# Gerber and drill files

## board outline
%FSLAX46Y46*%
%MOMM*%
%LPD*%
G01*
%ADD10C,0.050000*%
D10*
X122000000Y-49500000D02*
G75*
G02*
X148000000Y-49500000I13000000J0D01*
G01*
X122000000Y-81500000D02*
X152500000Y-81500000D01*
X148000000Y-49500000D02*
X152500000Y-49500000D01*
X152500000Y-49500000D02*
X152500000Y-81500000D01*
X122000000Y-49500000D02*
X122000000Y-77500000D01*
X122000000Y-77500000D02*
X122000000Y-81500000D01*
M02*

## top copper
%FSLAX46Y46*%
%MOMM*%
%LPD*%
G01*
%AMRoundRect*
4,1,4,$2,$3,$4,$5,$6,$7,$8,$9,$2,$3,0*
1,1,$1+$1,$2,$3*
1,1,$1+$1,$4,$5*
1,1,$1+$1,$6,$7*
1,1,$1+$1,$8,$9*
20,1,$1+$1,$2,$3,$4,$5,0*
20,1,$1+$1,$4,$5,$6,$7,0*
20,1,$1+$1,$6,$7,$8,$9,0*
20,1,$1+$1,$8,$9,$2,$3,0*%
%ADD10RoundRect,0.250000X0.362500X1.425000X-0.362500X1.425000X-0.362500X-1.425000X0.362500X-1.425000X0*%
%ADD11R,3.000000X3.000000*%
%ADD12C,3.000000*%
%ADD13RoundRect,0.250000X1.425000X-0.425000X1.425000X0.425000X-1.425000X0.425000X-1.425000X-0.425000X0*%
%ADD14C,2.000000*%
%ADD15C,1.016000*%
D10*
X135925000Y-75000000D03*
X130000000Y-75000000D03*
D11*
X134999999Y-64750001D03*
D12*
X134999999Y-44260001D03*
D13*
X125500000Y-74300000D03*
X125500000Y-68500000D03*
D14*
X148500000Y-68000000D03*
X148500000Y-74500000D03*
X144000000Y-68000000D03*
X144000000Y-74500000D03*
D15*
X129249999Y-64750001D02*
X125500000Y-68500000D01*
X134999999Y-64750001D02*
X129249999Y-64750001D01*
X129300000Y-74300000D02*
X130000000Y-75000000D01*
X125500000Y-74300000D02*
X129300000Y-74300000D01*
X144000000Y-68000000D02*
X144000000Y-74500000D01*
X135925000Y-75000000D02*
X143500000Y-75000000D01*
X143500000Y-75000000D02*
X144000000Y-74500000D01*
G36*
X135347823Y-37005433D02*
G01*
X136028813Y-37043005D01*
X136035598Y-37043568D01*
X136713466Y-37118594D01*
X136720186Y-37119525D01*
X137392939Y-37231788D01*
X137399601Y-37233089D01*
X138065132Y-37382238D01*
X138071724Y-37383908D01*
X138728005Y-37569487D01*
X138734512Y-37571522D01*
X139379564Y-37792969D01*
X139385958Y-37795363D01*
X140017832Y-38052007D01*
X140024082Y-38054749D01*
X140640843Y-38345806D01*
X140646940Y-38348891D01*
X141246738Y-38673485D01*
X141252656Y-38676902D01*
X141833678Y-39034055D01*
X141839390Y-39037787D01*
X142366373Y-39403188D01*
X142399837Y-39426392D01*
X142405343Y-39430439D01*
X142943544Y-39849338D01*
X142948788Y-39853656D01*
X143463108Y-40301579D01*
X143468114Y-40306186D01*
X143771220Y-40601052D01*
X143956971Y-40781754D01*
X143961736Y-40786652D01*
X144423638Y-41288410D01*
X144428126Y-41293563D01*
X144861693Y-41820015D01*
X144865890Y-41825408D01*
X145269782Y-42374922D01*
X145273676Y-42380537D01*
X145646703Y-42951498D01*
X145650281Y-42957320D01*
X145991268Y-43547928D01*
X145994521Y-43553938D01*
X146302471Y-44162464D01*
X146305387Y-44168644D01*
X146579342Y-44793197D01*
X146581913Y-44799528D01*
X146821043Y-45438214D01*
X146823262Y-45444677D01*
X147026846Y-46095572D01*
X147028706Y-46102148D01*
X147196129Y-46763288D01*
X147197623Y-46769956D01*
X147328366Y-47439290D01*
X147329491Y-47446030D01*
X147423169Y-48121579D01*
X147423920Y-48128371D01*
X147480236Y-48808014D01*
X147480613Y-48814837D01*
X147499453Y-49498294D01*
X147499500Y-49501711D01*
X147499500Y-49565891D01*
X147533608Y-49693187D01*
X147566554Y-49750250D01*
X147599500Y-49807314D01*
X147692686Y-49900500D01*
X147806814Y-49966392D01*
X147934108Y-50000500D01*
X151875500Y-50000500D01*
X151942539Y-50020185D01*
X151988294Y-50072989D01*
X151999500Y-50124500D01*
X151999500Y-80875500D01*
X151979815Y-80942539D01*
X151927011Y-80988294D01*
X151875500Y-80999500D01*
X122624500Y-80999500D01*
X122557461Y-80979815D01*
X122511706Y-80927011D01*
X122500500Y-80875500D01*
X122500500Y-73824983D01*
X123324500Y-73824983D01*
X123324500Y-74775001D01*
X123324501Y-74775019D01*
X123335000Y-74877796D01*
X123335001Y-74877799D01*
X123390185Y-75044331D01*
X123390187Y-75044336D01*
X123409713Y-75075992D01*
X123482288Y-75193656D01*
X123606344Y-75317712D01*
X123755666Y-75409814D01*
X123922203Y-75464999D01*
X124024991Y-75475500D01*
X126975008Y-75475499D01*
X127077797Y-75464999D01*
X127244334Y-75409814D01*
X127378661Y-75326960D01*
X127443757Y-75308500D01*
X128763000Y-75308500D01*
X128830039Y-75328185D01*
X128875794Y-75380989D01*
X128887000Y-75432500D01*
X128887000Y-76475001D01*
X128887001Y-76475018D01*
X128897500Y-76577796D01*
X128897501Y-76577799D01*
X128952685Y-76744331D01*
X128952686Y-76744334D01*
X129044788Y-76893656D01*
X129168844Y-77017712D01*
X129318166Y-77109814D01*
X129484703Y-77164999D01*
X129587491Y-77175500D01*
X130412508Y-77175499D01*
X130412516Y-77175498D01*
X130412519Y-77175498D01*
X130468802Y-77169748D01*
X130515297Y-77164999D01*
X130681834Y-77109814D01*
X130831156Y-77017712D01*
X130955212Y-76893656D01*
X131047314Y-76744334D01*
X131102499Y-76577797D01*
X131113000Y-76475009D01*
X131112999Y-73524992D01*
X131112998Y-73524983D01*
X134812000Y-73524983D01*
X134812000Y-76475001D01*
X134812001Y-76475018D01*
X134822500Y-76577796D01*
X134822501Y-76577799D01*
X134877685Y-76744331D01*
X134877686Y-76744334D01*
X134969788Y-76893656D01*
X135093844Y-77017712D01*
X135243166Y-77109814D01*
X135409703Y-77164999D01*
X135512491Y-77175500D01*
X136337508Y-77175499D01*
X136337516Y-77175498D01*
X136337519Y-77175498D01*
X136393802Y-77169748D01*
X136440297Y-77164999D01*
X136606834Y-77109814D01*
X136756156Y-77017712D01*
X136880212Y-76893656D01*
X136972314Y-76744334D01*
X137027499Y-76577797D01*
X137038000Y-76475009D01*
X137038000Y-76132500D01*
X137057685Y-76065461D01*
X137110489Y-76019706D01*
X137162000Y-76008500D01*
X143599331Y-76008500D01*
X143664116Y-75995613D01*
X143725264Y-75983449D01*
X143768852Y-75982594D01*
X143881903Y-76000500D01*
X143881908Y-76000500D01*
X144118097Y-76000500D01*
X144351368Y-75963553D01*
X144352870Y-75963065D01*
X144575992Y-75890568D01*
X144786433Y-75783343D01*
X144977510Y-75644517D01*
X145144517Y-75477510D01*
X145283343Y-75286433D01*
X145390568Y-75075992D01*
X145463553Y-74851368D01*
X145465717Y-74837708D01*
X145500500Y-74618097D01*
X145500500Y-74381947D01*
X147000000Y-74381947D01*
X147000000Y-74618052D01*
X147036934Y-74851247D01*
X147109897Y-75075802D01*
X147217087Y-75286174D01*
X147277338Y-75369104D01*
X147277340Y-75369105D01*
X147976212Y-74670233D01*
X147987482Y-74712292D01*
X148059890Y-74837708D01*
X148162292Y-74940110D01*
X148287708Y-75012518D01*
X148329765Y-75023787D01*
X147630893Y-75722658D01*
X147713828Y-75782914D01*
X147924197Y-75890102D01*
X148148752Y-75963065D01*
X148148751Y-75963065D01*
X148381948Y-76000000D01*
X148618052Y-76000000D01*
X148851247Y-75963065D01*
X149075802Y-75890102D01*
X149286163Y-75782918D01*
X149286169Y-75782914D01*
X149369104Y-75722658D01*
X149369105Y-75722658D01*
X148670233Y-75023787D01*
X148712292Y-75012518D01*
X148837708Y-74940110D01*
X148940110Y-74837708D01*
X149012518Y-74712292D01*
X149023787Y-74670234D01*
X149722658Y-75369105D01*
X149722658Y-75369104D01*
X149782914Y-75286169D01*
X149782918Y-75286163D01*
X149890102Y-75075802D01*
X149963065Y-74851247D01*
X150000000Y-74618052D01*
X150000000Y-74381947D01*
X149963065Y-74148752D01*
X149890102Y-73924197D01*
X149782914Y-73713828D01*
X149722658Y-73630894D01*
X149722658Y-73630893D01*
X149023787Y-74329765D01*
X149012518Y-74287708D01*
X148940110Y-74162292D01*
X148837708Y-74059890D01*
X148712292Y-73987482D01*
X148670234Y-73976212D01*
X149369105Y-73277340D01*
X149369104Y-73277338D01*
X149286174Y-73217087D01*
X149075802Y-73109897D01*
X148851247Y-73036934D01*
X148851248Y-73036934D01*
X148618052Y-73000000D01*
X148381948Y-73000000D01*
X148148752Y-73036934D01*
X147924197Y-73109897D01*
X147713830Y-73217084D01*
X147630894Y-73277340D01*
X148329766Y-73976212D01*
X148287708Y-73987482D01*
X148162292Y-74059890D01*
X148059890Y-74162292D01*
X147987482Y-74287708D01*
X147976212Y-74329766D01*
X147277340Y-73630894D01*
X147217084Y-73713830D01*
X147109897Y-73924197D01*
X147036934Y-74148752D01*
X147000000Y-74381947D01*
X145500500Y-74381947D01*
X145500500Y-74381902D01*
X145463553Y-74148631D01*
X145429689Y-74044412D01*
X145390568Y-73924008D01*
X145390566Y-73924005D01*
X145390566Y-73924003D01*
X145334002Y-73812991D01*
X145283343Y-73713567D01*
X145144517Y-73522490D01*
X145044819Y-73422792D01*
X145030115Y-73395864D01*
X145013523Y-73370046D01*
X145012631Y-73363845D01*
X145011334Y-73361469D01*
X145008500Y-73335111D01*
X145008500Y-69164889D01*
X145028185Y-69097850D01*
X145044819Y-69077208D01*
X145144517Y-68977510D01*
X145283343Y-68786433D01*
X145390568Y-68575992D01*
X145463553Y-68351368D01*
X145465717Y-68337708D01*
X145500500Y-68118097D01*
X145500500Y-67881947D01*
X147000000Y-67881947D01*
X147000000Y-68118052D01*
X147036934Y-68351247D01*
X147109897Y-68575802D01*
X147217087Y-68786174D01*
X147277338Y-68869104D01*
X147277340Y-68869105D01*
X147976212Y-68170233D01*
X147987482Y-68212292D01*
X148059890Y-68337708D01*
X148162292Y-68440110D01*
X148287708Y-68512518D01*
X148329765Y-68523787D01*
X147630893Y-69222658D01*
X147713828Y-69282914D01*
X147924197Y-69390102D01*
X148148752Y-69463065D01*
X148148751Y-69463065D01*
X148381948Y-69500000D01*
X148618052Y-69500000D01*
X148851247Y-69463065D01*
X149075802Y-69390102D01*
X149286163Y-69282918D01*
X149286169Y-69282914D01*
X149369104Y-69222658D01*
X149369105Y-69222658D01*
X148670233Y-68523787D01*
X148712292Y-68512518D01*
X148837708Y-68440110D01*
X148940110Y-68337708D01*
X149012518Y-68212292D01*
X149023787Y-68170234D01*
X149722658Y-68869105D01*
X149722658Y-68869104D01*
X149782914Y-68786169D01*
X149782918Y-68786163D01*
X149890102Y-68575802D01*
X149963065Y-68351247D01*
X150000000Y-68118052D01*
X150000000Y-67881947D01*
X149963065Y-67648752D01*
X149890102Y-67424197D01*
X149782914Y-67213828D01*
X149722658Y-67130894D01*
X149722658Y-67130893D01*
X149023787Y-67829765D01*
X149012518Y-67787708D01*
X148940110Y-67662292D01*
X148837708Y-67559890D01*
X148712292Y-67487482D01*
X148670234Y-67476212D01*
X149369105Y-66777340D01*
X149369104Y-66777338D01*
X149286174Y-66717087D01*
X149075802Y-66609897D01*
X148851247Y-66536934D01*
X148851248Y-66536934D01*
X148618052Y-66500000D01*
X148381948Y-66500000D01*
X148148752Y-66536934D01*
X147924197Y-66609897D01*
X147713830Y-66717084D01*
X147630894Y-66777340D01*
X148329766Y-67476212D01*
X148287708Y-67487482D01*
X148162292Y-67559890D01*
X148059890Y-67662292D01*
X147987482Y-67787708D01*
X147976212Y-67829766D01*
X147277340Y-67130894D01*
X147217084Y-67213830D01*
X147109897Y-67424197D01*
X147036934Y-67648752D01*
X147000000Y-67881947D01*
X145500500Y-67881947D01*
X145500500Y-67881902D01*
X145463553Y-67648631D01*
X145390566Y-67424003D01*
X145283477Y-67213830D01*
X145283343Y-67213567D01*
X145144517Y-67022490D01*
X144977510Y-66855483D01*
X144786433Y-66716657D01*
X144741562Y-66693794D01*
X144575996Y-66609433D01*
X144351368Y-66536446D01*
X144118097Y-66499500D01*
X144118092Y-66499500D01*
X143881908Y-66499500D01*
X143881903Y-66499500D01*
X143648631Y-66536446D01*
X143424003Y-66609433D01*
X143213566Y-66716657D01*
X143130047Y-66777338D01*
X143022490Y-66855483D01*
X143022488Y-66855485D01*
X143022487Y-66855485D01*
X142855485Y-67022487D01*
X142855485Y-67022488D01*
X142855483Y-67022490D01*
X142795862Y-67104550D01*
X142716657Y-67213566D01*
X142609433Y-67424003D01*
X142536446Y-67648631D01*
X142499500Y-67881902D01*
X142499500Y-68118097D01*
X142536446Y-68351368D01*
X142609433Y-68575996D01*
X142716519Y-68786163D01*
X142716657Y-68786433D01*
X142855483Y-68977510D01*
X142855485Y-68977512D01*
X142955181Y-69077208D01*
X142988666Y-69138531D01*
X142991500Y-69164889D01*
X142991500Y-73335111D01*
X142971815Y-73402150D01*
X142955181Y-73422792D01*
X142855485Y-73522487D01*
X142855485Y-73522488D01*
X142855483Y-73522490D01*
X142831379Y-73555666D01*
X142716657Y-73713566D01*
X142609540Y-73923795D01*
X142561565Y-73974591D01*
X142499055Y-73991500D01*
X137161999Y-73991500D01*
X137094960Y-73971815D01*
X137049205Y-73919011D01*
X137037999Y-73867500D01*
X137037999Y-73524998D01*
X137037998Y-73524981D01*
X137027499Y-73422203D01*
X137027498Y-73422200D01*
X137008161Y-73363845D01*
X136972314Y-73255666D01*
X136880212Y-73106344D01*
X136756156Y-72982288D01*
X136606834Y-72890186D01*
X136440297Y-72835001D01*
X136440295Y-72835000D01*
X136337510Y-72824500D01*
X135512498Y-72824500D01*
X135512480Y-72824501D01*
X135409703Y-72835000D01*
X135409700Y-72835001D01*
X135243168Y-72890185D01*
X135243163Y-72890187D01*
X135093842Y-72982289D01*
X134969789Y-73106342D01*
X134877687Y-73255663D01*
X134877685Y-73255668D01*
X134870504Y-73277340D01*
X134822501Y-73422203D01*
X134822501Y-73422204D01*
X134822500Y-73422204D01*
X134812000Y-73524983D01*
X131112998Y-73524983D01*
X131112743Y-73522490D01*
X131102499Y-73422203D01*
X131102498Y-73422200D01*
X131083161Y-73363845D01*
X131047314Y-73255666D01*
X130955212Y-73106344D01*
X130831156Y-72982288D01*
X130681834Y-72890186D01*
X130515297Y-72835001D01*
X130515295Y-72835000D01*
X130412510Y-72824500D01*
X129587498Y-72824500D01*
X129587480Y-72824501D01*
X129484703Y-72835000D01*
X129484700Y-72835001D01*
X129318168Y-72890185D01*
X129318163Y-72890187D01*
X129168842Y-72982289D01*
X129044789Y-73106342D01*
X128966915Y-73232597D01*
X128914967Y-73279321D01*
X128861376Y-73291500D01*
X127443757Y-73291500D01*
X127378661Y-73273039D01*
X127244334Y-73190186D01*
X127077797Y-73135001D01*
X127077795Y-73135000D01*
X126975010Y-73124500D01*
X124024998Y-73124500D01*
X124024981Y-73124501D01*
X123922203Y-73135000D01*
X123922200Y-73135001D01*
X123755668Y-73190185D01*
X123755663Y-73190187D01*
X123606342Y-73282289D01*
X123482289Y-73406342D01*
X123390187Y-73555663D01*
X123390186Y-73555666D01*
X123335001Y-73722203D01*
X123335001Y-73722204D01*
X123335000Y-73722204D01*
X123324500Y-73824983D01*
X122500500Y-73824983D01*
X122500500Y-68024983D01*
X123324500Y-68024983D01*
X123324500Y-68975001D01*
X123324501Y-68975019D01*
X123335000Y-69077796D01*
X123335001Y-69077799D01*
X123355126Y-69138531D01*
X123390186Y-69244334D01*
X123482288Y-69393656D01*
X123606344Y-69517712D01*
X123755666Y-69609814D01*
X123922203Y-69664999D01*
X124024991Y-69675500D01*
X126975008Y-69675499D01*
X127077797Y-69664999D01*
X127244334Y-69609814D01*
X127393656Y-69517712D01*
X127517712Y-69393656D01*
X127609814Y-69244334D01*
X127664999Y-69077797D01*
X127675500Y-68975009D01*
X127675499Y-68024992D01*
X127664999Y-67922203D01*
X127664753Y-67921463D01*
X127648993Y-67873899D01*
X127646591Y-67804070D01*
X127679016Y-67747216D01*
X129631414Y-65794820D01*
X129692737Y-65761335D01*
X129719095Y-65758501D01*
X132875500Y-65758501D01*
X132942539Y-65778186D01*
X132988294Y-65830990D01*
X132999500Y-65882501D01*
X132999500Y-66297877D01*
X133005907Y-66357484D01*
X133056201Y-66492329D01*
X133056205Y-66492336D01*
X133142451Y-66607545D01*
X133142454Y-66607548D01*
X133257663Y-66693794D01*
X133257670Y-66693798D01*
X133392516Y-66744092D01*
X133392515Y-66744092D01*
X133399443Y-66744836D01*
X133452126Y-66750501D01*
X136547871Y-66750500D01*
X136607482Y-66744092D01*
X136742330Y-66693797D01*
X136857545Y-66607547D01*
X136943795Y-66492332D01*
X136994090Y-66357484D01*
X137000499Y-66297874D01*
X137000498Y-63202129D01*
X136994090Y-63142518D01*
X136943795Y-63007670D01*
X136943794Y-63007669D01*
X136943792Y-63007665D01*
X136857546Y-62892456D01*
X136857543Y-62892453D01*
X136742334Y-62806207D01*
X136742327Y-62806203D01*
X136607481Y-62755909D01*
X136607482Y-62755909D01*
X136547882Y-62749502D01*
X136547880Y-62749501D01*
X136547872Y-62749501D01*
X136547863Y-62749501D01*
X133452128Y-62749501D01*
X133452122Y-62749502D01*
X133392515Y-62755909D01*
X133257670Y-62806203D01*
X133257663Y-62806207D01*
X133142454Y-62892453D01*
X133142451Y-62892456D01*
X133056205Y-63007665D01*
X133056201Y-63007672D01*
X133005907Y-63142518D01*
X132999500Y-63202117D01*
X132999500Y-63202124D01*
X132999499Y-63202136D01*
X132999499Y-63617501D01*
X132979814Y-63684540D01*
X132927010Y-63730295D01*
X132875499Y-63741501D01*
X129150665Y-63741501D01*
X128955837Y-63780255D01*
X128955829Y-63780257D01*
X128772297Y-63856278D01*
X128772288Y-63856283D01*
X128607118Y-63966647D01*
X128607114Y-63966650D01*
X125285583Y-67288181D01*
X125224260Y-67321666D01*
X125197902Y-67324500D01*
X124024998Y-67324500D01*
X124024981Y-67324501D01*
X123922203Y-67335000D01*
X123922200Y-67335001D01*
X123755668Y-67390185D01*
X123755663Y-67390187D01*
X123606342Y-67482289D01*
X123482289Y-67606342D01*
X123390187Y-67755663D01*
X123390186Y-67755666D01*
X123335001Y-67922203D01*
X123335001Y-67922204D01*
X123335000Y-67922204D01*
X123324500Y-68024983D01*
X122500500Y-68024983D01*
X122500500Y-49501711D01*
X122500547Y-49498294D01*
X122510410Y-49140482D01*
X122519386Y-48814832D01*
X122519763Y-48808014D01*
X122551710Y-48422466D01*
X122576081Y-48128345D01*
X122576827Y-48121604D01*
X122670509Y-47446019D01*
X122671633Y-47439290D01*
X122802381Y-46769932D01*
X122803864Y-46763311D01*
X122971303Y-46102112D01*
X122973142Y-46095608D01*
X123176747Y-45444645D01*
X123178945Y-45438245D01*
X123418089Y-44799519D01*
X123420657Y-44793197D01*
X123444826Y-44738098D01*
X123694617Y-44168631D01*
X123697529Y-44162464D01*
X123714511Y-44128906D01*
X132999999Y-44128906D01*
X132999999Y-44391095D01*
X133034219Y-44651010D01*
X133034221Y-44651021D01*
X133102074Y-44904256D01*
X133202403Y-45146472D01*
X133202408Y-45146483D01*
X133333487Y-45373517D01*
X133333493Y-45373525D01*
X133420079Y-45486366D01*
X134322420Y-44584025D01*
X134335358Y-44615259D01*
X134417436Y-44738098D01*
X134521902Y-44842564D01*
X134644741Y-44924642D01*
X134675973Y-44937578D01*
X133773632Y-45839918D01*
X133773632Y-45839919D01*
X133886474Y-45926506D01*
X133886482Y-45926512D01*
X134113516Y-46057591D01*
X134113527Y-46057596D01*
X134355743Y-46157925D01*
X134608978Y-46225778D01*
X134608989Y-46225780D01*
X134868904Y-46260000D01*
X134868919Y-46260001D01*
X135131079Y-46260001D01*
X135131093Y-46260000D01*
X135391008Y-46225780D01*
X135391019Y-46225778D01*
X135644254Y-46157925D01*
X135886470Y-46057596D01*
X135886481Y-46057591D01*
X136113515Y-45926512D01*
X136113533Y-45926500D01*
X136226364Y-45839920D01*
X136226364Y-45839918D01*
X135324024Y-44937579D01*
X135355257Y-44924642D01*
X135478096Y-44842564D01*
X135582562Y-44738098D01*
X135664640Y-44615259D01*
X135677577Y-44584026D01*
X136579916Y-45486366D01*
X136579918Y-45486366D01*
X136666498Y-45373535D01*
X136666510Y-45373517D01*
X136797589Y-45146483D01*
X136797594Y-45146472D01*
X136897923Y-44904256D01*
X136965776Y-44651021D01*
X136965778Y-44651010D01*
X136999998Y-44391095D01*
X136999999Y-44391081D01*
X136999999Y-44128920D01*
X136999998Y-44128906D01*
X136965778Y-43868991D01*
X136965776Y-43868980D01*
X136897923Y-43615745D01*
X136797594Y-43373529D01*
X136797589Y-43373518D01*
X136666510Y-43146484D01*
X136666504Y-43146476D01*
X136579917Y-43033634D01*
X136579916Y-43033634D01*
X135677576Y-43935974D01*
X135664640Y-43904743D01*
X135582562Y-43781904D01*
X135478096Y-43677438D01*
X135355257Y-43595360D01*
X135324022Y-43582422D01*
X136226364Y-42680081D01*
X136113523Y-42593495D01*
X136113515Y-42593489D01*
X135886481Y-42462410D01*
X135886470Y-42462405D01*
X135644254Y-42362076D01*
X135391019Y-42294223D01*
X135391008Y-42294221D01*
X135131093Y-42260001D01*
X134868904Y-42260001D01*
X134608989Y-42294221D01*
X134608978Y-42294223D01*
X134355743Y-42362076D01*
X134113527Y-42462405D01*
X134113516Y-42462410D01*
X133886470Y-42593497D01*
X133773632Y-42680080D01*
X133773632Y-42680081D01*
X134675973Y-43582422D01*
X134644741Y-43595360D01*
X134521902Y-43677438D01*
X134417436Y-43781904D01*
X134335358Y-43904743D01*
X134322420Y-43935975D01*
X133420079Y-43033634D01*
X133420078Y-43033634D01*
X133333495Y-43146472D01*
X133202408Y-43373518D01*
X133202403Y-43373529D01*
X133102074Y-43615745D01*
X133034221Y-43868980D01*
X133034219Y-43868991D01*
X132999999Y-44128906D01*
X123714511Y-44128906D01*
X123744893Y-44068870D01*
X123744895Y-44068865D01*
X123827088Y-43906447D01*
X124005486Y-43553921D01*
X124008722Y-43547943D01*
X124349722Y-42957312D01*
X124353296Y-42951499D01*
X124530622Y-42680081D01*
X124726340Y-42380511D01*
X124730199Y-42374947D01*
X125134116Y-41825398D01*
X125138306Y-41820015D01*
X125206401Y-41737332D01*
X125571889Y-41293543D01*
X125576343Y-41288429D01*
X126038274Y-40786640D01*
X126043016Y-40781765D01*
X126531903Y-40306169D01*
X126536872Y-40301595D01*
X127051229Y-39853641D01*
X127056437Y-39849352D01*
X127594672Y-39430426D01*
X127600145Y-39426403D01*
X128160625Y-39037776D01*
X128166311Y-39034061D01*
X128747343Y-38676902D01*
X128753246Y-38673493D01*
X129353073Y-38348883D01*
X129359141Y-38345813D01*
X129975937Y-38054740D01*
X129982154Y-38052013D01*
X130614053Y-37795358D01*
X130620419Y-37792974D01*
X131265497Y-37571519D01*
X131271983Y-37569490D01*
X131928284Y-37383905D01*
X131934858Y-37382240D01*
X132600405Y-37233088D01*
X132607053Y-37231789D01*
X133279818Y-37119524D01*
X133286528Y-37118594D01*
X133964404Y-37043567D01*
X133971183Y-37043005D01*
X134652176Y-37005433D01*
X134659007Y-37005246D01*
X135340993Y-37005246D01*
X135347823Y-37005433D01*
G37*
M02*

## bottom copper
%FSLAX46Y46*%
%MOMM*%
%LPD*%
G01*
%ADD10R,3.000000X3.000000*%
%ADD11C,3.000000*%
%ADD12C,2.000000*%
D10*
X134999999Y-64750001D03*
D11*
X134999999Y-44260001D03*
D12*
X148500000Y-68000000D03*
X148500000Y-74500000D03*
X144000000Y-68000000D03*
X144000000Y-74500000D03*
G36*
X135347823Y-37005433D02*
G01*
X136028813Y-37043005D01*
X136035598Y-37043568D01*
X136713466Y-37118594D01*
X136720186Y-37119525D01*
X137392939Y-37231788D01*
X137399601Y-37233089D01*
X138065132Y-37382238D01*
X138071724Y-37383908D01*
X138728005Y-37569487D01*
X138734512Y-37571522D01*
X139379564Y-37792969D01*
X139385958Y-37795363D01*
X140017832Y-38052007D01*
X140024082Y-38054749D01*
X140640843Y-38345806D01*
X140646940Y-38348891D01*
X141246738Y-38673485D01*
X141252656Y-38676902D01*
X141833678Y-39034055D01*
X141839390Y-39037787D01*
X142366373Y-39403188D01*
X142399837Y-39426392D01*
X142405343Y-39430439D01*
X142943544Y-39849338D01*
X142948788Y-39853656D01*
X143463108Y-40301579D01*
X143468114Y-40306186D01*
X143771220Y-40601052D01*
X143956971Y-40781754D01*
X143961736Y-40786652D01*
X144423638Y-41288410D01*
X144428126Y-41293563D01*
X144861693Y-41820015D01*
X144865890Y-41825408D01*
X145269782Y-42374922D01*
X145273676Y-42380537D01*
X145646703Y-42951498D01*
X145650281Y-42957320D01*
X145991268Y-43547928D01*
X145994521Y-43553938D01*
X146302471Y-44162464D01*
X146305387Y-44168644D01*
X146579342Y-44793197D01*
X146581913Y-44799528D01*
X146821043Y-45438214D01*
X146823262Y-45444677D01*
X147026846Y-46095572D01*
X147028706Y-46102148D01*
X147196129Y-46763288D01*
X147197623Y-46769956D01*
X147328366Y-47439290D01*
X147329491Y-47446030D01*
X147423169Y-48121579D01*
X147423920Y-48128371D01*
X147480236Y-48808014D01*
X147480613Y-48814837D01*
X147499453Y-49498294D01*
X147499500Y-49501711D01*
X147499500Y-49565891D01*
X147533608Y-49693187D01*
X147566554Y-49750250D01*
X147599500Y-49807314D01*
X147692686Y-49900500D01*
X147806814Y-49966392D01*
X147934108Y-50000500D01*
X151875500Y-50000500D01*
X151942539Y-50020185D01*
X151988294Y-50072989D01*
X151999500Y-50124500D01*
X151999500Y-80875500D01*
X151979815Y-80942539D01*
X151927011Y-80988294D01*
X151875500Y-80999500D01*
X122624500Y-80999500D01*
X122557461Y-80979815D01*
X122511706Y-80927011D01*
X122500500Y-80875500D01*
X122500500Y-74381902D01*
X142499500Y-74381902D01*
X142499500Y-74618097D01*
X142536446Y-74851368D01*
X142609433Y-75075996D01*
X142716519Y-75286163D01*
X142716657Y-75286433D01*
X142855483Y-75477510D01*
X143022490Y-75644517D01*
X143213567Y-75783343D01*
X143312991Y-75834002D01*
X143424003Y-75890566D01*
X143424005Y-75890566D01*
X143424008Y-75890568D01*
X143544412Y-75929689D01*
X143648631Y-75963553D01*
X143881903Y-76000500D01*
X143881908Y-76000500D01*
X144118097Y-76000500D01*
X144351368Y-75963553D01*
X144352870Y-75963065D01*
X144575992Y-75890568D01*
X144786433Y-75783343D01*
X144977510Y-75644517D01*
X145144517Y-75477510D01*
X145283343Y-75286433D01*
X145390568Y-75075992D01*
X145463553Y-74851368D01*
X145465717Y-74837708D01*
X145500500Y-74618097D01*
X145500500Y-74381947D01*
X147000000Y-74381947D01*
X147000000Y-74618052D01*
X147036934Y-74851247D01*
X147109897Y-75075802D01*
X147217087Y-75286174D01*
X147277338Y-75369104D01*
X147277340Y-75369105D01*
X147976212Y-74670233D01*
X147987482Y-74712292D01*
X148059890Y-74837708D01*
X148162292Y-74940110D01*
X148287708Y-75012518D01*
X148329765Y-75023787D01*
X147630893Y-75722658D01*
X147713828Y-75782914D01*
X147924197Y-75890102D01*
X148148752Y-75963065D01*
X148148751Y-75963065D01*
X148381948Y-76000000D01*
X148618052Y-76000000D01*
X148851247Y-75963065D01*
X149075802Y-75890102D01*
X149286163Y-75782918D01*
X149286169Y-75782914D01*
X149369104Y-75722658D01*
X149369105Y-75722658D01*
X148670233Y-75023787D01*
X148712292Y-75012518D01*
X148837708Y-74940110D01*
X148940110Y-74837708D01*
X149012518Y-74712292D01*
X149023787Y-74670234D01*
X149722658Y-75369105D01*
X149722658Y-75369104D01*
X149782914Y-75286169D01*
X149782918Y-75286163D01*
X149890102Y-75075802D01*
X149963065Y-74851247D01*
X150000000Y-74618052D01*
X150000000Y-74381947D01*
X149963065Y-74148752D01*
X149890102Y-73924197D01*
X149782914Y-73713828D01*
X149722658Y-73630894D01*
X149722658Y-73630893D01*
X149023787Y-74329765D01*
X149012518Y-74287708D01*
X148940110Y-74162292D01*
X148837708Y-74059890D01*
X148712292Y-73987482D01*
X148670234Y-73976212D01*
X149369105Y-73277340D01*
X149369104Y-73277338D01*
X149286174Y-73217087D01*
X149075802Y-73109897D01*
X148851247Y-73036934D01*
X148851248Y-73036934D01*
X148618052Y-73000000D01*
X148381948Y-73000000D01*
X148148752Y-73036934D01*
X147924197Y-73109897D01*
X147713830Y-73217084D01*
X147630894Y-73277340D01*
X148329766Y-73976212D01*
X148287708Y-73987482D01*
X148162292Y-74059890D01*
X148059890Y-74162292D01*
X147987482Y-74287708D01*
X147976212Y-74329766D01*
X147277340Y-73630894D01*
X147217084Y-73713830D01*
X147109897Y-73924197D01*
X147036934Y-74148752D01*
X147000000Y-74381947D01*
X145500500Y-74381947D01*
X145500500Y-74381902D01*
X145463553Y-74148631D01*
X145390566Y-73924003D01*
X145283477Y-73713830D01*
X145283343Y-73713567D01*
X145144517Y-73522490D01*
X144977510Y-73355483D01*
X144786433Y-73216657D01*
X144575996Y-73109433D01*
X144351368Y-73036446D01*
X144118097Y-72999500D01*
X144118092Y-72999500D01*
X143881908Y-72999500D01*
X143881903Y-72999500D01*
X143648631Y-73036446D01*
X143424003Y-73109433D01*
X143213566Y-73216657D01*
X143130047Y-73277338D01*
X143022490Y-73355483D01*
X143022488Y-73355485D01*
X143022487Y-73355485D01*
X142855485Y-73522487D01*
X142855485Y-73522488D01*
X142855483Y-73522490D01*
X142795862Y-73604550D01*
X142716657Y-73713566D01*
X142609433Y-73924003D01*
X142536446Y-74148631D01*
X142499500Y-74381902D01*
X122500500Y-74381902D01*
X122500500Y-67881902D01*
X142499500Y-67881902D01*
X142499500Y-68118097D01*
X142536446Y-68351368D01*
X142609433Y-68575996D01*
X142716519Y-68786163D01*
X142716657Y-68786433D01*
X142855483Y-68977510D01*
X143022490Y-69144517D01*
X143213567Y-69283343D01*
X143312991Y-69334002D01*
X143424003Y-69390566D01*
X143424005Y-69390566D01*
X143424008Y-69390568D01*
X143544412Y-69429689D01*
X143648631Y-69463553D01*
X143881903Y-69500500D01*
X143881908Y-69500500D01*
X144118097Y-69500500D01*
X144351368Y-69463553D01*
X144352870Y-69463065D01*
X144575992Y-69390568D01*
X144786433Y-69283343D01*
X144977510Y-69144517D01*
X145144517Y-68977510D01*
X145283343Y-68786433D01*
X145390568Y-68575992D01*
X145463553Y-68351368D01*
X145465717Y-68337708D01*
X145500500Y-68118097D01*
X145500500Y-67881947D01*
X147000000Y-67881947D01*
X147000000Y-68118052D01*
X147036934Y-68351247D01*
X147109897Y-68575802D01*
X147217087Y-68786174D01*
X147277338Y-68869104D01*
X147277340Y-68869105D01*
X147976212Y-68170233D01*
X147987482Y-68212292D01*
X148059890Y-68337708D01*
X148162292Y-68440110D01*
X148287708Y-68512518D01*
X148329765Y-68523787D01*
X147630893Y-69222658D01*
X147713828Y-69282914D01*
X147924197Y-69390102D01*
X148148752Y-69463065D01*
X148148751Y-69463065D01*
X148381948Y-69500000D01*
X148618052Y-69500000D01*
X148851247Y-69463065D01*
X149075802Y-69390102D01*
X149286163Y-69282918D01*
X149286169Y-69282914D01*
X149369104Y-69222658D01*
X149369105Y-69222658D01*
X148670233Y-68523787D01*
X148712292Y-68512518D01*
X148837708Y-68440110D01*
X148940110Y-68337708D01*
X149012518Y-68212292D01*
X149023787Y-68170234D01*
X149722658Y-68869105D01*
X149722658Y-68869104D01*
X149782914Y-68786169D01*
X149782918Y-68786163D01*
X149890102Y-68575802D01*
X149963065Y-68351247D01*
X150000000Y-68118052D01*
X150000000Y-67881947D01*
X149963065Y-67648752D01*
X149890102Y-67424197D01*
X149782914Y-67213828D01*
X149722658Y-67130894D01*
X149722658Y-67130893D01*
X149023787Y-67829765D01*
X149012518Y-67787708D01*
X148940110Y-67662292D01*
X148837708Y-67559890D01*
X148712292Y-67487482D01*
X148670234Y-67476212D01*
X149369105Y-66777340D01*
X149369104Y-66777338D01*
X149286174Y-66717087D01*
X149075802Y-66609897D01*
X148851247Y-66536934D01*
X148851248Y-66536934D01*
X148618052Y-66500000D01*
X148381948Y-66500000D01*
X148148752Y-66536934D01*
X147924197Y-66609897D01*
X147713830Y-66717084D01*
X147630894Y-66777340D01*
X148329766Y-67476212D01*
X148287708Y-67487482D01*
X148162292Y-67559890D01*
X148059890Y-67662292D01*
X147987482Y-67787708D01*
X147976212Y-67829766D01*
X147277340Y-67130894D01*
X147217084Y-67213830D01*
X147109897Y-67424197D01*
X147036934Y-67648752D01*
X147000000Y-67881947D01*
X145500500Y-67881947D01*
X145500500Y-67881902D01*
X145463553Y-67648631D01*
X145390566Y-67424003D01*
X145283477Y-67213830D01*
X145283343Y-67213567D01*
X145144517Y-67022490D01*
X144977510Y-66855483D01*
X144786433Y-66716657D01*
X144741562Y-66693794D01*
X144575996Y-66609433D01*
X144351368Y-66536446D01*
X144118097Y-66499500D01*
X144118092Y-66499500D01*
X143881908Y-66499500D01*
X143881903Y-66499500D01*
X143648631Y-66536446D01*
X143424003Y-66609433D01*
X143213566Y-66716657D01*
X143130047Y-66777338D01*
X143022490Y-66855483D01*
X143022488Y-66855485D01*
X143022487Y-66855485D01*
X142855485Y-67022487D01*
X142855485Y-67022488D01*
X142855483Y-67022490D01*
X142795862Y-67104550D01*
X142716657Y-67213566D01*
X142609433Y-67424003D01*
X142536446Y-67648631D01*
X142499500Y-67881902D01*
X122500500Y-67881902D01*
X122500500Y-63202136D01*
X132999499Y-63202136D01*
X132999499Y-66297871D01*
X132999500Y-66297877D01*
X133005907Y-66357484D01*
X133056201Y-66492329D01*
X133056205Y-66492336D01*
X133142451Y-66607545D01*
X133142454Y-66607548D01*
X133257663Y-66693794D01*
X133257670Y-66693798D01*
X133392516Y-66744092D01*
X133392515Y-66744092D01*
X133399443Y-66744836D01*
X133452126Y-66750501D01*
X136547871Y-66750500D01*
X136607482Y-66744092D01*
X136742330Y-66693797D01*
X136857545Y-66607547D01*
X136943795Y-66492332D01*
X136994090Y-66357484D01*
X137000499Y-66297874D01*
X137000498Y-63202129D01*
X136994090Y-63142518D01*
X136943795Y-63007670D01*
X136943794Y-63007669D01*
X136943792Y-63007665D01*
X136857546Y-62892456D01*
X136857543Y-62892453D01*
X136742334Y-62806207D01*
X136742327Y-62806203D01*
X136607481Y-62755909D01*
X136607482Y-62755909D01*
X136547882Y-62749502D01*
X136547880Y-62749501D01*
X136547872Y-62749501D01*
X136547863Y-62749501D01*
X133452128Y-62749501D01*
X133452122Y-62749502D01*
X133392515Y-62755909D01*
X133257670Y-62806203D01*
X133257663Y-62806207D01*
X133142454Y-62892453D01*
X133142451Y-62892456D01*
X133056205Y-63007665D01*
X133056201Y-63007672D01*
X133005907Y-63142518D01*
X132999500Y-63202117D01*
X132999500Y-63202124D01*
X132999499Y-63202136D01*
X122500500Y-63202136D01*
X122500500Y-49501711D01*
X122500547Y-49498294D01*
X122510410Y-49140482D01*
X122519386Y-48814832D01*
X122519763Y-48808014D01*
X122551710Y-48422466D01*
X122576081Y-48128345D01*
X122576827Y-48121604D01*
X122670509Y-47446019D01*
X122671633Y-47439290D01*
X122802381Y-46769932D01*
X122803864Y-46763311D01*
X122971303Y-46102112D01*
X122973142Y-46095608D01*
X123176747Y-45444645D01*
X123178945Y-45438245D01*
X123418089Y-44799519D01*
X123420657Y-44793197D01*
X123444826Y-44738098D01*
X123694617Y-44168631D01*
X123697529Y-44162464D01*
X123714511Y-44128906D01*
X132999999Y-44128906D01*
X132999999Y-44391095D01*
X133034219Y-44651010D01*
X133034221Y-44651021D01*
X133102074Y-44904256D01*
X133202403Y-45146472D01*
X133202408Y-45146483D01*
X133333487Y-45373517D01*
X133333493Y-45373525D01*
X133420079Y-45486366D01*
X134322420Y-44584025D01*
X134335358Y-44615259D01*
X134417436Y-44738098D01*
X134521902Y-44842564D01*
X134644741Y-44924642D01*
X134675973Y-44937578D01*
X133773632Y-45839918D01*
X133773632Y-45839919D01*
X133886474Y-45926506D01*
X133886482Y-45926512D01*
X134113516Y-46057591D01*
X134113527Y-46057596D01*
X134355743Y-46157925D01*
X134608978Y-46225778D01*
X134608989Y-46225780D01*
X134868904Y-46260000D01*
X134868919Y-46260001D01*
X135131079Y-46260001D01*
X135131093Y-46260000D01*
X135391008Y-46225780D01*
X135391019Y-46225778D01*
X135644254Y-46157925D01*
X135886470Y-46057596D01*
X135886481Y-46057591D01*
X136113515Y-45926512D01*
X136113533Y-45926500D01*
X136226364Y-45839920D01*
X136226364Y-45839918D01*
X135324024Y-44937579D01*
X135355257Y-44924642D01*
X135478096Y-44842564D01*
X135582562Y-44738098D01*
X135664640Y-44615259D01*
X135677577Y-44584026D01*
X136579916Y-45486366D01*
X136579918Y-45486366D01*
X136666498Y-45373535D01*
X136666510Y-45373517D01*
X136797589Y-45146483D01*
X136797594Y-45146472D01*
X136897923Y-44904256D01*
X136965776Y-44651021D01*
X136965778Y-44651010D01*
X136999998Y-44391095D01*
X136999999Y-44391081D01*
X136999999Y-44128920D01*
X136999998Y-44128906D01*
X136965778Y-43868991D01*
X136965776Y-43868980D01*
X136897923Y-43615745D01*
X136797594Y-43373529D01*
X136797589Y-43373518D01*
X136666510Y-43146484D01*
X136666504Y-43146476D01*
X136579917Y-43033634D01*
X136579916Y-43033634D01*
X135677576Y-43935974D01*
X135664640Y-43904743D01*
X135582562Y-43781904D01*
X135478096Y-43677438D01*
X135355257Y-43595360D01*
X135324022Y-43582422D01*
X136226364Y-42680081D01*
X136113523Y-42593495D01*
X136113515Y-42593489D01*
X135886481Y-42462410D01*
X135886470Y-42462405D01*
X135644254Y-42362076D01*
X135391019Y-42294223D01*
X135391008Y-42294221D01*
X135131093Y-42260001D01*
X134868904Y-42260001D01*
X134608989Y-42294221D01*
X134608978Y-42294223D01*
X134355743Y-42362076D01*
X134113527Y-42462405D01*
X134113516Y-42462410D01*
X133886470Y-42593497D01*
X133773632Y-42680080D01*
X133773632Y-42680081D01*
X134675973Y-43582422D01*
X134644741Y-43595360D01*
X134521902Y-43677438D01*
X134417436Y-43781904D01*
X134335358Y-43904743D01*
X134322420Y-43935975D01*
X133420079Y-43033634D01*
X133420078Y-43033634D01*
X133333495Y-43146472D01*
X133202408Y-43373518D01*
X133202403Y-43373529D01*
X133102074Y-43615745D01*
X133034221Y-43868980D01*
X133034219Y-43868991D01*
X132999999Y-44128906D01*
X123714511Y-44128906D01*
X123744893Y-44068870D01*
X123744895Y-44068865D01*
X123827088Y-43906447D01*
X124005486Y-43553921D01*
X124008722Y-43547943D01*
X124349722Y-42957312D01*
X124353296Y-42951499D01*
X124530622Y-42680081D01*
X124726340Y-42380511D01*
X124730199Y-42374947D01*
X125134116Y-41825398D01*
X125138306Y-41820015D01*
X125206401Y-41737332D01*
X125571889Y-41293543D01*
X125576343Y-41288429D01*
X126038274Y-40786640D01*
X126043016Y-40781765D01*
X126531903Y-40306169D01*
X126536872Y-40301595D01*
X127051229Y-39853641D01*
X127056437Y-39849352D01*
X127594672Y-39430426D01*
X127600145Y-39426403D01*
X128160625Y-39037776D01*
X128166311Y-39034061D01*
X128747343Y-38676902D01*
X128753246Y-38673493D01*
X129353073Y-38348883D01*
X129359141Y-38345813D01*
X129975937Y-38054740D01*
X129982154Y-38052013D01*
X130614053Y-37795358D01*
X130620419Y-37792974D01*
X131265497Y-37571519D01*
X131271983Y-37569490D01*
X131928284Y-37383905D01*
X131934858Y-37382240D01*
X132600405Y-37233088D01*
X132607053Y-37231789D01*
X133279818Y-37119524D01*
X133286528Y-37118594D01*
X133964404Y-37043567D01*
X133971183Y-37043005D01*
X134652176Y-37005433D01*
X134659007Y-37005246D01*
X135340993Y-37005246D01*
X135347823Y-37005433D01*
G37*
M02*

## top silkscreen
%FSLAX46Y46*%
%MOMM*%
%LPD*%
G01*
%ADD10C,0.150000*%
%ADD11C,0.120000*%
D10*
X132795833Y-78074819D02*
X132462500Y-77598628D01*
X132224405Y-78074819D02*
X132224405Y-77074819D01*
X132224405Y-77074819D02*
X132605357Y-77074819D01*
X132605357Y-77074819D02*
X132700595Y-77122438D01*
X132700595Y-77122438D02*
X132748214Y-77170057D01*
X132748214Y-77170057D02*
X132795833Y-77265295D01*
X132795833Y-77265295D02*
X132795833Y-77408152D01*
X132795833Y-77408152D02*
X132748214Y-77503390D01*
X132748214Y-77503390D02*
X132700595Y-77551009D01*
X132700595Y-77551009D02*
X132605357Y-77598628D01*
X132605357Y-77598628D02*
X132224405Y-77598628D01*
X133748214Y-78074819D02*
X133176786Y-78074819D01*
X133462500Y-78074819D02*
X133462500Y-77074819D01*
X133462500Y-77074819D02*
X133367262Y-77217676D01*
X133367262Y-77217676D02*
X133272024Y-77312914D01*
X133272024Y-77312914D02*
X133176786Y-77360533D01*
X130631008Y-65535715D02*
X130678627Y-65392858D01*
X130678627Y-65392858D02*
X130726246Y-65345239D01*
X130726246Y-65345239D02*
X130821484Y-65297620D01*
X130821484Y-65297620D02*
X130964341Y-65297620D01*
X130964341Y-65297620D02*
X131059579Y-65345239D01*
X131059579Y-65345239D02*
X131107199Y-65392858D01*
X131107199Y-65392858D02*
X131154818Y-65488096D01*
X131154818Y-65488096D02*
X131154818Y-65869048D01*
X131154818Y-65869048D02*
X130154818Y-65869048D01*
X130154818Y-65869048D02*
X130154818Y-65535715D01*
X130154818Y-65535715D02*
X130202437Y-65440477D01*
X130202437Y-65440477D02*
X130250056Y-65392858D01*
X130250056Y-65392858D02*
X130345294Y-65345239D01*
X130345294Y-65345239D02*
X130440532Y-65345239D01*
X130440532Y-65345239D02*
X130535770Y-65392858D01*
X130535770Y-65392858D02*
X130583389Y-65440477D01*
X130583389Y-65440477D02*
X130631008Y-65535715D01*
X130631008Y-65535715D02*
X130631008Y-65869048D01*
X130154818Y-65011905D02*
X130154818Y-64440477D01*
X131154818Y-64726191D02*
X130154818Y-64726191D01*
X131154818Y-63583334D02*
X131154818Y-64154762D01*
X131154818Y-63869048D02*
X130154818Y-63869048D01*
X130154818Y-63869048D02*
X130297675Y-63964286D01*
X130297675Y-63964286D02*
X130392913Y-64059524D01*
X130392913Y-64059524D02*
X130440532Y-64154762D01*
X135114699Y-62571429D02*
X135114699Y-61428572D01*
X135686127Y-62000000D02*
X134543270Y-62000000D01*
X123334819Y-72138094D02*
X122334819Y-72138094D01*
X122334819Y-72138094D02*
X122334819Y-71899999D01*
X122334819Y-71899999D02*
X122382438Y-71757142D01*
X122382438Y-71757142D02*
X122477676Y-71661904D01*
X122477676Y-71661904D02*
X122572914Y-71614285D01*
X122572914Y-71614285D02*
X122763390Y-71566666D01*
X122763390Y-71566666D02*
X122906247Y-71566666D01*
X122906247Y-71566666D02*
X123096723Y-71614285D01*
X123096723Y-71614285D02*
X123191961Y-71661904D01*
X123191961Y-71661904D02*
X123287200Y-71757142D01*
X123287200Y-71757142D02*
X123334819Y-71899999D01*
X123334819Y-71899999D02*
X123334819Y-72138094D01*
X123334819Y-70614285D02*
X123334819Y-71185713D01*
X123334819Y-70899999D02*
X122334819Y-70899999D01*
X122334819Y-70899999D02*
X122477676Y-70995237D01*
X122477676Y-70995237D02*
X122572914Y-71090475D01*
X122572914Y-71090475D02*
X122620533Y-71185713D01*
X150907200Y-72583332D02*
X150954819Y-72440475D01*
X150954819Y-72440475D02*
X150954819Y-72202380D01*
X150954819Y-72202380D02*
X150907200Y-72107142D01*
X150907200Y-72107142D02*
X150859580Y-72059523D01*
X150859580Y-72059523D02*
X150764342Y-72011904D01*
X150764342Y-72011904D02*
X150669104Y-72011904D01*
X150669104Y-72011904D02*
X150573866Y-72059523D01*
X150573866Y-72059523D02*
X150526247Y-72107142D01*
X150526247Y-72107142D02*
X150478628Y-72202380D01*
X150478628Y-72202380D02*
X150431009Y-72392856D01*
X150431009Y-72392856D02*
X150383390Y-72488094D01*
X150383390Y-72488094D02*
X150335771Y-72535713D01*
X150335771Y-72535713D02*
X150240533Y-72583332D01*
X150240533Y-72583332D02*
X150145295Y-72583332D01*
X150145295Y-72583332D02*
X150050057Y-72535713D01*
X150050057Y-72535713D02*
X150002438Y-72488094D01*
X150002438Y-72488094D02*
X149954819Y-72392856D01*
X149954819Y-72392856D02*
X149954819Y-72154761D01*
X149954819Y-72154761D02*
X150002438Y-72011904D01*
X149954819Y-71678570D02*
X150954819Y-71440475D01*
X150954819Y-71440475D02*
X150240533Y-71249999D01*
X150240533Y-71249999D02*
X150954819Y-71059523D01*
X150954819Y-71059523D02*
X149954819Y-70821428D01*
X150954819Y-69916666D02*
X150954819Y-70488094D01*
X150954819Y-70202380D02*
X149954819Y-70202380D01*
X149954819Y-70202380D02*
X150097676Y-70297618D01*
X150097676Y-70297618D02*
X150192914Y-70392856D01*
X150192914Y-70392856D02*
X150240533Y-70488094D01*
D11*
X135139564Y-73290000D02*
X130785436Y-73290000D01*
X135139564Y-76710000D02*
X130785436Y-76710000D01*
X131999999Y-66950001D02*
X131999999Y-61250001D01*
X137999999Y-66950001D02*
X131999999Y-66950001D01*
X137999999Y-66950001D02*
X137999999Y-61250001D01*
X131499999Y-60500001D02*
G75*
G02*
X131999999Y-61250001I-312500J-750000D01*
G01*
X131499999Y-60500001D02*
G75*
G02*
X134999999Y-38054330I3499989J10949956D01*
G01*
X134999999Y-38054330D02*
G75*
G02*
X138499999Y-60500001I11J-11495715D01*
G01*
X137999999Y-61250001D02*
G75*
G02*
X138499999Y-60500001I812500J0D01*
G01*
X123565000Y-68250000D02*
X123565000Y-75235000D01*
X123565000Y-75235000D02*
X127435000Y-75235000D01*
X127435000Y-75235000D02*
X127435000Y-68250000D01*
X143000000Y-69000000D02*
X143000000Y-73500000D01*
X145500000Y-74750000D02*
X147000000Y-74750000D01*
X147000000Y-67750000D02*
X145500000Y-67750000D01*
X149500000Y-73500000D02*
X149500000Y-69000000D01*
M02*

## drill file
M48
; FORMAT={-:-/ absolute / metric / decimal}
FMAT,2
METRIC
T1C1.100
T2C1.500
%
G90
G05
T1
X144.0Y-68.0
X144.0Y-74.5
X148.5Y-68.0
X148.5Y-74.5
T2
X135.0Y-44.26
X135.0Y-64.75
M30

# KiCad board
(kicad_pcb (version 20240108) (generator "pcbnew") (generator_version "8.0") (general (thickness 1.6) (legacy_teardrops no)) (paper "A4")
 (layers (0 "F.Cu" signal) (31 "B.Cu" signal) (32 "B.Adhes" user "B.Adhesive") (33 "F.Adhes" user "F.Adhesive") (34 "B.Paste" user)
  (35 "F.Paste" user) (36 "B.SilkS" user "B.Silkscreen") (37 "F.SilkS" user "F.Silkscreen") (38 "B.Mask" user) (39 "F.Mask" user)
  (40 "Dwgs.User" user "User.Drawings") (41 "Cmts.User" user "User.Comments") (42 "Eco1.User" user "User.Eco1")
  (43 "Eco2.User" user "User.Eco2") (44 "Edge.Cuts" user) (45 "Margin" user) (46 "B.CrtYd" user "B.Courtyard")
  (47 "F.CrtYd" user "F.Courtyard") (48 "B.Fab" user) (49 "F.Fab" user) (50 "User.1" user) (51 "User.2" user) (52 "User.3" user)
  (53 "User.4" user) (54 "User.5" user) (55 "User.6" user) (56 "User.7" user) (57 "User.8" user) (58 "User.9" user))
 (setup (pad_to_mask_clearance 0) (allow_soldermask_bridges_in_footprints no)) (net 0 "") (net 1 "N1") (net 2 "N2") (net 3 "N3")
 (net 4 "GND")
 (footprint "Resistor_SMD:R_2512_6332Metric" (layer "F.Cu") (at 132.9625 75 180)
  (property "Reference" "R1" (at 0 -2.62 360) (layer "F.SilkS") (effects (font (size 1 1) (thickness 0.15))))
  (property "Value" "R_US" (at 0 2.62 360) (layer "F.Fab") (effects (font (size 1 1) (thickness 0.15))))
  (fp_line (start -2.177064 1.71) (end 2.177064 1.71) (stroke (width 0.12) (type solid)) (layer "F.SilkS"))
  (fp_line (start -2.177064 -1.71) (end 2.177064 -1.71) (stroke (width 0.12) (type solid)) (layer "F.SilkS"))
  (pad "1" smd roundrect (at -2.9625 0 180) (size 1.225 3.35) (layers "F.Cu" "F.Paste" "F.Mask") (roundrect_rratio 0.204082) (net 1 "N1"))
  (pad "2" smd roundrect (at 2.9625 0 180) (size 1.225 3.35) (layers "F.Cu" "F.Paste" "F.Mask") (roundrect_rratio 0.204082) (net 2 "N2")))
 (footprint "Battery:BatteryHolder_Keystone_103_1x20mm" (layer "F.Cu") (at 134.999999 64.750001 90)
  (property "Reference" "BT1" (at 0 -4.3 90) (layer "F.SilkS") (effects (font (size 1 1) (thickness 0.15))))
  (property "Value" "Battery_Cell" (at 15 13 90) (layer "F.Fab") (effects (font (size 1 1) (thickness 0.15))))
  (fp_line (start -2.2 -3) (end 3.5 -3) (stroke (width 0.12) (type solid)) (layer "F.SilkS"))
  (fp_line (start -2.2 3) (end -2.2 -3) (stroke (width 0.12) (type solid)) (layer "F.SilkS"))
  (fp_line (start -2.2 3) (end 3.5 3) (stroke (width 0.12) (type solid)) (layer "F.SilkS"))
  (fp_arc (start 4.25 -3.5) (mid 3.950694 -3.136459) (end 3.5 -3) (stroke (width 0.12) (type solid)) (layer "F.SilkS"))
  (fp_arc (start 4.25 -3.5) (mid 16.971103 -11.358466) (end 26.695671 0) (stroke (width 0.12) (type solid)) (layer "F.SilkS"))
  (fp_arc (start 26.695671 0) (mid 16.971103 11.358466) (end 4.25 3.5) (stroke (width 0.12) (type solid)) (layer "F.SilkS"))
  (fp_arc (start 3.5 3) (mid 3.950694 3.136459) (end 4.25 3.5) (stroke (width 0.12) (type solid)) (layer "F.SilkS"))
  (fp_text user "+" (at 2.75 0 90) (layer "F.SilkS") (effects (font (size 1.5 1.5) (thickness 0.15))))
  (pad "1" thru_hole rect (at 0 0 90) (size 3 3) (drill 1.5) (layers "*.Cu" "*.Mask") (remove_unused_layers no) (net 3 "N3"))
  (pad "2" thru_hole circle (at 20.49 0 90) (size 3 3) (drill 1.5) (layers "*.Cu" "*.Mask") (remove_unused_layers no) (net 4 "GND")))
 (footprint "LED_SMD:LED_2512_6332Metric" (layer "F.Cu") (at 125.5 71.4 90)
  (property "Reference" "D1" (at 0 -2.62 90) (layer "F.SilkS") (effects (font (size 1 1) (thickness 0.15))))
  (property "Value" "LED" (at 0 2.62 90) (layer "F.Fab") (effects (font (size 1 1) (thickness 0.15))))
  (fp_line (start 3.15 -1.935) (end -3.835 -1.935) (stroke (width 0.12) (type solid)) (layer "F.SilkS"))
  (fp_line (start -3.835 -1.935) (end -3.835 1.935) (stroke (width 0.12) (type solid)) (layer "F.SilkS"))
  (fp_line (start -3.835 1.935) (end 3.15 1.935) (stroke (width 0.12) (type solid)) (layer "F.SilkS"))
  (pad "1" smd roundrect (at -2.9 0 90) (size 1.35 3.35) (layers "F.Cu" "F.Paste" "F.Mask") (roundrect_rratio 0.185185) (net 2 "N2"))
  (pad "2" smd roundrect (at 2.9 0 90) (size 1.35 3.35) (layers "F.Cu" "F.Paste" "F.Mask") (roundrect_rratio 0.185185) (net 3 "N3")))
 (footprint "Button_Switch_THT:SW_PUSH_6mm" (layer "F.Cu") (at 148.5 68 -90)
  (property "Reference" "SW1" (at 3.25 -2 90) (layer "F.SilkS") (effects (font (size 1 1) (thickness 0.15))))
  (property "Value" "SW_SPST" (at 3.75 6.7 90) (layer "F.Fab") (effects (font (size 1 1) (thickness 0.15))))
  (fp_line (start 1 5.5) (end 5.5 5.5) (stroke (width 0.12) (type solid)) (layer "F.SilkS"))
  (fp_line (start 6.75 3) (end 6.75 1.5) (stroke (width 0.12) (type solid)) (layer "F.SilkS"))
  (fp_line (start -0.25 1.5) (end -0.25 3) (stroke (width 0.12) (type solid)) (layer "F.SilkS"))
  (fp_line (start 5.5 -1) (end 1 -1) (stroke (width 0.12) (type solid)) (layer "F.SilkS"))
  (pad "1" thru_hole circle (at 0 0) (size 2 2) (drill 1.1) (layers "*.Cu" "*.Mask") (remove_unused_layers no) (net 4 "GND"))
  (pad "1" thru_hole circle (at 6.5 0) (size 2 2) (drill 1.1) (layers "*.Cu" "*.Mask") (remove_unused_layers no) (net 4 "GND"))
  (pad "2" thru_hole circle (at 0 4.5) (size 2 2) (drill 1.1) (layers "*.Cu" "*.Mask") (remove_unused_layers no) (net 1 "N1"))
  (pad "2" thru_hole circle (at 6.5 4.5) (size 2 2) (drill 1.1) (layers "*.Cu" "*.Mask") (remove_unused_layers no) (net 1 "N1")))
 (gr_arc (start 122 49.5) (mid 135 36.5) (end 148 49.5) (stroke (width 0.05) (type default)) (layer "Edge.Cuts"))
 (gr_line (start 122 81.5) (end 152.5 81.5) (stroke (width 0.05) (type default)) (layer "Edge.Cuts"))
 (gr_line (start 148 49.5) (end 152.5 49.5) (stroke (width 0.05) (type default)) (layer "Edge.Cuts"))
 (gr_line (start 152.5 49.5) (end 152.5 81.5) (stroke (width 0.05) (type default)) (layer "Edge.Cuts"))
 (gr_line (start 122 49.5) (end 122 77.5) (stroke (width 0.05) (type default)) (layer "Edge.Cuts"))
 (gr_line (start 122 77.5) (end 122 81.5) (stroke (width 0.05) (type default)) (layer "Edge.Cuts"))
 (segment (start 129.249999 64.750001) (end 125.5 68.5) (width 1.016) (layer "F.Cu") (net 3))
 (segment (start 134.999999 64.750001) (end 129.249999 64.750001) (width 1.016) (layer "F.Cu") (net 3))
 (segment (start 129.3 74.3) (end 130 75) (width 1.016) (layer "F.Cu") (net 2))
 (segment (start 125.5 74.3) (end 129.3 74.3) (width 1.016) (layer "F.Cu") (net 2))
 (segment (start 144 68) (end 144 74.5) (width 1.016) (layer "F.Cu") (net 1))
 (segment (start 135.925 75) (end 143.5 75) (width 1.016) (layer "F.Cu") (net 1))
 (segment (start 143.5 75) (end 144 74.5) (width 1.016) (layer "F.Cu") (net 1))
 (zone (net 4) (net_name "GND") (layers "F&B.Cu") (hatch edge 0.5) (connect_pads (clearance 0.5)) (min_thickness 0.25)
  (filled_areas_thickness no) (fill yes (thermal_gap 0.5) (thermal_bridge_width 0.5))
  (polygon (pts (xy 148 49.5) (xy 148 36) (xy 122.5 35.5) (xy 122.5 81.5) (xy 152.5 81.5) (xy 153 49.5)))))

